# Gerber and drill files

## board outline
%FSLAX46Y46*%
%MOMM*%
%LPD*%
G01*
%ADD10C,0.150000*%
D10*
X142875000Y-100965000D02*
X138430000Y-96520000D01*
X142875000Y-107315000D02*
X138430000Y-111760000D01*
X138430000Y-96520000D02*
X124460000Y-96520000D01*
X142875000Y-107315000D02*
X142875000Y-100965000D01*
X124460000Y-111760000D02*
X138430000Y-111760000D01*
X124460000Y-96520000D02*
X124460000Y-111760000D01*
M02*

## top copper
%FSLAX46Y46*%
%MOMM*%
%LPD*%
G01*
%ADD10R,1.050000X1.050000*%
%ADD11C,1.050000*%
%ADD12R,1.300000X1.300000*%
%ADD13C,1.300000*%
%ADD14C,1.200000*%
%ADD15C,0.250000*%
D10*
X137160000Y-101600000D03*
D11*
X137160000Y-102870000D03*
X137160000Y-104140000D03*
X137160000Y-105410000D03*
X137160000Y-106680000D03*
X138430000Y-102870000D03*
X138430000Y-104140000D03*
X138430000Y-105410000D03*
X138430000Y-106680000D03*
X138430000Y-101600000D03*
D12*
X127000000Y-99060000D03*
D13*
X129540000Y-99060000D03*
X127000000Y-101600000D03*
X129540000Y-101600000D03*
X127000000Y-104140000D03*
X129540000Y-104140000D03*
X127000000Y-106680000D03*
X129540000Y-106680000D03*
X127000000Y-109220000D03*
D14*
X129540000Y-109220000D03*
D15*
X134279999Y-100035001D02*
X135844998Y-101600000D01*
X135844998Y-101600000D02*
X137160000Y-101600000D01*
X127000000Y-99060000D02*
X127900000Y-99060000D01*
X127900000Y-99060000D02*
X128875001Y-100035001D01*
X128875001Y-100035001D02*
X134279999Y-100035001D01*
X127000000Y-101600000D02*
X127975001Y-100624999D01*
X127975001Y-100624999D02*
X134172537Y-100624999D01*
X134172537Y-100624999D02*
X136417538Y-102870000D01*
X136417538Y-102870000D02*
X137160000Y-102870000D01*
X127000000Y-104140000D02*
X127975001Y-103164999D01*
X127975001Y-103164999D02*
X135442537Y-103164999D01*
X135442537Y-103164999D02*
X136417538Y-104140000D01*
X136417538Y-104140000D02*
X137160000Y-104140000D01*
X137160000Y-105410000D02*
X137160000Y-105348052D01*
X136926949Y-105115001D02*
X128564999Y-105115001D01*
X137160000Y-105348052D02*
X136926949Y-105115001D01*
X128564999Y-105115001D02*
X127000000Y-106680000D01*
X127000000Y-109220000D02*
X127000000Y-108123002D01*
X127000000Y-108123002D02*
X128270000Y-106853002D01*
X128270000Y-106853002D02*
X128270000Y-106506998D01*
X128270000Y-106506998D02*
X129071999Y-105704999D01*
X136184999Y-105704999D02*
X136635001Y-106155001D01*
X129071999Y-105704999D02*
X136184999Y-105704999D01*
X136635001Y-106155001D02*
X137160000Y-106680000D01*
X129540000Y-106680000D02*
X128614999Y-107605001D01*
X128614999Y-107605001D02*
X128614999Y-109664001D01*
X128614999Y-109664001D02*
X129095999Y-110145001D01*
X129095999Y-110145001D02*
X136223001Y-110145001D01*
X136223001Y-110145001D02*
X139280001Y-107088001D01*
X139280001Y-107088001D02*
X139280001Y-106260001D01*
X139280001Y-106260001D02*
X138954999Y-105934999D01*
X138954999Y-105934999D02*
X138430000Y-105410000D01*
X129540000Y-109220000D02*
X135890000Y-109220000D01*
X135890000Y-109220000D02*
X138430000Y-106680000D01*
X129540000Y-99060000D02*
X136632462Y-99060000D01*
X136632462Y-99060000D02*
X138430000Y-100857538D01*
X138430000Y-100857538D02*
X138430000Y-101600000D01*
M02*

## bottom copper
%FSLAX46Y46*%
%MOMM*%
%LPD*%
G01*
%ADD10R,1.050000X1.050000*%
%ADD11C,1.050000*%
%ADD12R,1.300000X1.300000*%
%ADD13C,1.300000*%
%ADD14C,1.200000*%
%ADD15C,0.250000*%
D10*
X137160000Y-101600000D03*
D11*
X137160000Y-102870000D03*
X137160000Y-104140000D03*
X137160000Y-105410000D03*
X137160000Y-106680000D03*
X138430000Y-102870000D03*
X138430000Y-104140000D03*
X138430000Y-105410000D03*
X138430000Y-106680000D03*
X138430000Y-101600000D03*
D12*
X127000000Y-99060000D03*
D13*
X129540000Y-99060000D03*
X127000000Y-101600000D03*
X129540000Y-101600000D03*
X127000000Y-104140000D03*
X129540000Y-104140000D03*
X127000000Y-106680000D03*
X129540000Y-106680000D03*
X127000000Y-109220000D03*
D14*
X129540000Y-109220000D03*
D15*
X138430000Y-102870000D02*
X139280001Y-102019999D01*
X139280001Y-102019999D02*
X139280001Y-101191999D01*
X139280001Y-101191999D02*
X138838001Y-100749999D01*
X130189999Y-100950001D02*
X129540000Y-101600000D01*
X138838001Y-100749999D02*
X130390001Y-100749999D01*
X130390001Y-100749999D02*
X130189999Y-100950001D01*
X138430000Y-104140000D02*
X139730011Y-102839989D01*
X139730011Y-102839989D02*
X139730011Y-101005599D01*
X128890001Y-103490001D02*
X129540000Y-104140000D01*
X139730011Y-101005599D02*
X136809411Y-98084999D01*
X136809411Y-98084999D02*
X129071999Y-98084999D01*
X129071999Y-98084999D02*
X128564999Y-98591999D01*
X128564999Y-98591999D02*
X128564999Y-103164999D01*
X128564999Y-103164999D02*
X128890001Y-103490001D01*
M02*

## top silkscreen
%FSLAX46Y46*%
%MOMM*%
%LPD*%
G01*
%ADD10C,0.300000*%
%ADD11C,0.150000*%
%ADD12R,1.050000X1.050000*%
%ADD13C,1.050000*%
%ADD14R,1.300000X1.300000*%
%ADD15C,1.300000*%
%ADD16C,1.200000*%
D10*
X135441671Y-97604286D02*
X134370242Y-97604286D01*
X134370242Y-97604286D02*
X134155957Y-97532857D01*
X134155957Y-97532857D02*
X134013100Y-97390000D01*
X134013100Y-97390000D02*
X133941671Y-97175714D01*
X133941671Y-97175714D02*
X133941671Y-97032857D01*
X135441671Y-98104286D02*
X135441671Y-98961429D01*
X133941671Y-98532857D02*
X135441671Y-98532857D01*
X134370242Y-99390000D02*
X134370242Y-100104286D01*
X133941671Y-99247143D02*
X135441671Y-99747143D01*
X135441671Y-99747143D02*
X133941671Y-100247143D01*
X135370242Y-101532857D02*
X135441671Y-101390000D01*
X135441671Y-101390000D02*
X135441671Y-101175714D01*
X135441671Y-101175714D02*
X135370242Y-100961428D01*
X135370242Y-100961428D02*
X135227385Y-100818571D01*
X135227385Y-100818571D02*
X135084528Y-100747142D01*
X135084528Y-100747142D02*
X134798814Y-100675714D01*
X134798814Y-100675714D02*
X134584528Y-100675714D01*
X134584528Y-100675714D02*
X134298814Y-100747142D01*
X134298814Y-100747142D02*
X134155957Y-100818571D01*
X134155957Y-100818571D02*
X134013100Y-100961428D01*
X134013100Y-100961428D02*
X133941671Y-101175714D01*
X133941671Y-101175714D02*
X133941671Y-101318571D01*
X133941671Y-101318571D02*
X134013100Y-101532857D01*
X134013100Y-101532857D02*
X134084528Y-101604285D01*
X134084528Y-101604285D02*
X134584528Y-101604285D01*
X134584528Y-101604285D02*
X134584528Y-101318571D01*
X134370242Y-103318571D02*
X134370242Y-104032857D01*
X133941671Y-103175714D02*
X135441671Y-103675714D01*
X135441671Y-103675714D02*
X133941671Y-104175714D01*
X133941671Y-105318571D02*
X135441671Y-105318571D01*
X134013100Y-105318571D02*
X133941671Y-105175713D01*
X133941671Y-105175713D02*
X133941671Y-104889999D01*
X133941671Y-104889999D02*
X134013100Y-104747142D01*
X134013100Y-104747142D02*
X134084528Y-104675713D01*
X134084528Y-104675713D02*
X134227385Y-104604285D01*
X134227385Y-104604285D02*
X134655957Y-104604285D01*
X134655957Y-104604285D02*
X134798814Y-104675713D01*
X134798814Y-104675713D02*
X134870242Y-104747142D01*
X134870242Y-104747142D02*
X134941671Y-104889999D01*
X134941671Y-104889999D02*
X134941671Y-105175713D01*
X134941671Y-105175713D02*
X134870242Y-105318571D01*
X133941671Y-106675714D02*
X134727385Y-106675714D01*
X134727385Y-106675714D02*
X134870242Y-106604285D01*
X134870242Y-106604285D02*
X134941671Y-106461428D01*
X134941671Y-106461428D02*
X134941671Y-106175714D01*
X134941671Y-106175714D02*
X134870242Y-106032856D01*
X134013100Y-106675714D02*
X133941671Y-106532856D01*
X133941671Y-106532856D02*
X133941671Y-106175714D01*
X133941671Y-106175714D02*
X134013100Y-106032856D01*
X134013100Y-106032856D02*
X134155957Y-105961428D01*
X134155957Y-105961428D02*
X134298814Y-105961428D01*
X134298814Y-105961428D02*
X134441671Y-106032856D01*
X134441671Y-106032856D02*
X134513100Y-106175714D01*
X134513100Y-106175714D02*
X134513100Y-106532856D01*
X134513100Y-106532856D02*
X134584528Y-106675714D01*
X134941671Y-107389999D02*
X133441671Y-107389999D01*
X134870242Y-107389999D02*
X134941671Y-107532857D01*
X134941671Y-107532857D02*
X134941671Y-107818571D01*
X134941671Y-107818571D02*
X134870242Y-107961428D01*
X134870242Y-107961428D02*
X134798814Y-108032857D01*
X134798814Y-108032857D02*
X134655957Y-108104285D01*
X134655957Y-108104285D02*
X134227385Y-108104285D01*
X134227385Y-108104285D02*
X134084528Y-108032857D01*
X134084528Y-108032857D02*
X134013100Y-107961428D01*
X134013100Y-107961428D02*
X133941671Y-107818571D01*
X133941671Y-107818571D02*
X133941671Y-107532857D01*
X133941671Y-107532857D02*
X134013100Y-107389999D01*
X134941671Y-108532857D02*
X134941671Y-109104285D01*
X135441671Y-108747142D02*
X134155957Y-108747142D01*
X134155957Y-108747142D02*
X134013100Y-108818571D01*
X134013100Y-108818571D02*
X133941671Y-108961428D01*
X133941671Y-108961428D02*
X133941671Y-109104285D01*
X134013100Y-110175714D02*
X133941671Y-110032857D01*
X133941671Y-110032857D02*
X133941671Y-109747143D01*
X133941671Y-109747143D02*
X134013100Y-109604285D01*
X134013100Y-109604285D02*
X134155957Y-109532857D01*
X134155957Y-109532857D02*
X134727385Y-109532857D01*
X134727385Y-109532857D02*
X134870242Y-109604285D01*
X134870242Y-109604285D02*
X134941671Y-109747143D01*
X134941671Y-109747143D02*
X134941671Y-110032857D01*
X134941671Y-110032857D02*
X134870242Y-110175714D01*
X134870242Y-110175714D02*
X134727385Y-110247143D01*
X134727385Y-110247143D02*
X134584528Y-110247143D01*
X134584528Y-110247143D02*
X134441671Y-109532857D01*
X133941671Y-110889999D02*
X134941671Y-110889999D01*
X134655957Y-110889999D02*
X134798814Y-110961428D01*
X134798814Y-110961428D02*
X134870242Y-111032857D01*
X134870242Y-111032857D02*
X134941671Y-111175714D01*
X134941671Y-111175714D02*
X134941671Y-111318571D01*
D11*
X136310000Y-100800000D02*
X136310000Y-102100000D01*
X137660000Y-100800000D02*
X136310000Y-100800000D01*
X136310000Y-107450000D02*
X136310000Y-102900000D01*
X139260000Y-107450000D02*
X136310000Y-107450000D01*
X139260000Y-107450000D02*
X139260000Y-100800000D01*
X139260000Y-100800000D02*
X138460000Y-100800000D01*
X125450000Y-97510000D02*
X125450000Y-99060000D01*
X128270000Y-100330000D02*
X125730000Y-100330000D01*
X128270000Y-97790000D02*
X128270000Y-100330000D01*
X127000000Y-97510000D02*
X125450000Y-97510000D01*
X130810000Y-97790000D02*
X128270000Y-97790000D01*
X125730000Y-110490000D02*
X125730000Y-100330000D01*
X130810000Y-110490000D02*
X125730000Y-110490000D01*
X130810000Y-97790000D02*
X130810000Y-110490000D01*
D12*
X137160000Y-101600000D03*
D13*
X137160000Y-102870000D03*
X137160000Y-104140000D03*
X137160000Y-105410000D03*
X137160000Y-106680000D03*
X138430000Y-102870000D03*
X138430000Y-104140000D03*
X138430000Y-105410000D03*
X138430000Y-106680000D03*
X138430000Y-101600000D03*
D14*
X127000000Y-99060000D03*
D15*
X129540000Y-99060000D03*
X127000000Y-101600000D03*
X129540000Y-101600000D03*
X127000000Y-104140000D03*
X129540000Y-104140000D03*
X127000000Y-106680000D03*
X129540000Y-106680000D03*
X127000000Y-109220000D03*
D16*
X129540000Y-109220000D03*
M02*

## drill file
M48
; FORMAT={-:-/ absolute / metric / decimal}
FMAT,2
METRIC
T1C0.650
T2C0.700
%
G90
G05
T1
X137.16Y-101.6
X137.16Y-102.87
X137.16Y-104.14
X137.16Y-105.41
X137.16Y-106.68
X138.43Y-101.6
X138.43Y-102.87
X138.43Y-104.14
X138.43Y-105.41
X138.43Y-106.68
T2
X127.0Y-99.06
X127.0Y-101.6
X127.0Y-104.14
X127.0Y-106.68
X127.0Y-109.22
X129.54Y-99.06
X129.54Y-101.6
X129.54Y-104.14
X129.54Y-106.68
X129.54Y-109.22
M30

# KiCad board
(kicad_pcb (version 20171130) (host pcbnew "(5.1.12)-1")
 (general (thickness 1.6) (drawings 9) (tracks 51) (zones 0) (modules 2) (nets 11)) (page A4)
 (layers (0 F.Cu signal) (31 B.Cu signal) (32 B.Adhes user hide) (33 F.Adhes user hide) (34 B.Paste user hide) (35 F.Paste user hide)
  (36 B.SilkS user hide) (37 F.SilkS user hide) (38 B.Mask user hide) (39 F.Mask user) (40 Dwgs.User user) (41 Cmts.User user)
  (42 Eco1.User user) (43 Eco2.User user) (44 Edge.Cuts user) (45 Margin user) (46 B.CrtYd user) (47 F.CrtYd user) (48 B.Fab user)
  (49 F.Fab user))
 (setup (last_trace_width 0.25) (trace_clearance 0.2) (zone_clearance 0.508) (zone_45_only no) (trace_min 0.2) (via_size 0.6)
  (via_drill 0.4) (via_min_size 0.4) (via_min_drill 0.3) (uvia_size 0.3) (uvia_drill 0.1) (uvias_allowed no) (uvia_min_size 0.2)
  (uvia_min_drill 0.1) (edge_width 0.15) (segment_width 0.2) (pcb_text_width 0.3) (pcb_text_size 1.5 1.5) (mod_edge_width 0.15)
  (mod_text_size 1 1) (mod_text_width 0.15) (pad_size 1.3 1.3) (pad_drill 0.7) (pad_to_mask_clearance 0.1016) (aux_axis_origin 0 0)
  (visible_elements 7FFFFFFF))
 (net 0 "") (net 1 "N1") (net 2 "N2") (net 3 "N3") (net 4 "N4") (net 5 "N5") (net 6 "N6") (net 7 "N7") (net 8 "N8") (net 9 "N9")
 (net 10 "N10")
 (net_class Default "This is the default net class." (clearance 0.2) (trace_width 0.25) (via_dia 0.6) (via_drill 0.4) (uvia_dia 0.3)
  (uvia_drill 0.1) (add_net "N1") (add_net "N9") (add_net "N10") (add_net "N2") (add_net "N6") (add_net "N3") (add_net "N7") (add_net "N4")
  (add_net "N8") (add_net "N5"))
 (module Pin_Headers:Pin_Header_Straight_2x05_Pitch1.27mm (layer F.Cu) (at 137.16 101.6)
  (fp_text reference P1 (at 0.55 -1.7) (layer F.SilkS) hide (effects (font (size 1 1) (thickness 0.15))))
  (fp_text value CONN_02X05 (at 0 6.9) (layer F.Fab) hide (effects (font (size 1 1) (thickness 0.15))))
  (fp_line (start -0.85 -0.8) (end -0.85 0.5) (layer F.SilkS) (width 0.15))
  (fp_line (start 0.5 -0.8) (end -0.85 -0.8) (layer F.SilkS) (width 0.15))
  (fp_line (start -0.85 5.85) (end -0.85 1.3) (layer F.SilkS) (width 0.15))
  (fp_line (start 2.1 5.85) (end -0.85 5.85) (layer F.SilkS) (width 0.15))
  (fp_line (start 2.1 5.85) (end 2.1 -0.8) (layer F.SilkS) (width 0.15))
  (fp_line (start 2.1 -0.8) (end 1.3 -0.8) (layer F.SilkS) (width 0.15))
  (pad 1 thru_hole rect (at 0 0) (size 1.05 1.05) (drill 0.65) (layers *.Cu *.Mask F.SilkS) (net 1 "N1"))
  (pad 3 thru_hole circle (at 0 1.27) (size 1.05 1.05) (drill 0.65) (layers *.Cu *.Mask F.SilkS) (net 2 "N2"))
  (pad 5 thru_hole circle (at 0 2.54) (size 1.05 1.05) (drill 0.65) (layers *.Cu *.Mask F.SilkS) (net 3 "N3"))
  (pad 7 thru_hole circle (at 0 3.81) (size 1.05 1.05) (drill 0.65) (layers *.Cu *.Mask F.SilkS) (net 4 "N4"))
  (pad 9 thru_hole circle (at 0 5.08) (size 1.05 1.05) (drill 0.65) (layers *.Cu *.Mask F.SilkS) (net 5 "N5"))
  (pad 4 thru_hole circle (at 1.27 1.27) (size 1.05 1.05) (drill 0.65) (layers *.Cu *.Mask F.SilkS) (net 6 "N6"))
  (pad 6 thru_hole circle (at 1.27 2.54) (size 1.05 1.05) (drill 0.65) (layers *.Cu *.Mask F.SilkS) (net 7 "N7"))
  (pad 8 thru_hole circle (at 1.27 3.81) (size 1.05 1.05) (drill 0.65) (layers *.Cu *.Mask F.SilkS) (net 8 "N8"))
  (pad 10 thru_hole circle (at 1.27 5.08) (size 1.05 1.05) (drill 0.65) (layers *.Cu *.Mask F.SilkS) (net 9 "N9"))
  (pad 2 thru_hole circle (at 1.27 0) (size 1.05 1.05) (drill 0.65) (layers *.Cu *.Mask F.SilkS) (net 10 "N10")))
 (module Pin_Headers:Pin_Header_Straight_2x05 (layer F.Cu) (at 127 99.06)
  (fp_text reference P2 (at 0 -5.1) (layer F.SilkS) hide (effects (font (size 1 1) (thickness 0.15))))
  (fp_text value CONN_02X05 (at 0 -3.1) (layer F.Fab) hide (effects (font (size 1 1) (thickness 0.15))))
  (fp_line (start -1.55 -1.55) (end -1.55 0) (layer F.SilkS) (width 0.15))
  (fp_line (start 1.27 1.27) (end -1.27 1.27) (layer F.SilkS) (width 0.15))
  (fp_line (start 1.27 -1.27) (end 1.27 1.27) (layer F.SilkS) (width 0.15))
  (fp_line (start 0 -1.55) (end -1.55 -1.55) (layer F.SilkS) (width 0.15))
  (fp_line (start 3.81 -1.27) (end 1.27 -1.27) (layer F.SilkS) (width 0.15))
  (fp_line (start -1.27 11.43) (end -1.27 1.27) (layer F.SilkS) (width 0.15))
  (fp_line (start 3.81 11.43) (end -1.27 11.43) (layer F.SilkS) (width 0.15))
  (fp_line (start 3.81 -1.27) (end 3.81 11.43) (layer F.SilkS) (width 0.15))
  (pad 1 thru_hole rect (at 0 0) (size 1.3 1.3) (drill 0.7) (layers *.Cu *.Mask F.SilkS) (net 1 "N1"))
  (pad 2 thru_hole circle (at 2.54 0) (size 1.3 1.3) (drill 0.7) (layers *.Cu *.Mask F.SilkS) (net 10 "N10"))
  (pad 3 thru_hole circle (at 0 2.54) (size 1.3 1.3) (drill 0.7) (layers *.Cu *.Mask F.SilkS) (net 2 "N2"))
  (pad 4 thru_hole circle (at 2.54 2.54) (size 1.3 1.3) (drill 0.7) (layers *.Cu *.Mask F.SilkS) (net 6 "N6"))
  (pad 5 thru_hole circle (at 0 5.08) (size 1.3 1.3) (drill 0.7) (layers *.Cu *.Mask F.SilkS) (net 3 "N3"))
  (pad 6 thru_hole circle (at 2.54 5.08) (size 1.3 1.3) (drill 0.7) (layers *.Cu *.Mask F.SilkS) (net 7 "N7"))
  (pad 7 thru_hole circle (at 0 7.62) (size 1.3 1.3) (drill 0.7) (layers *.Cu *.Mask F.SilkS) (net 4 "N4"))
  (pad 8 thru_hole circle (at 2.54 7.62) (size 1.3 1.3) (drill 0.7) (layers *.Cu *.Mask F.SilkS) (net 8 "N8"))
  (pad 9 thru_hole circle (at 0 10.16) (size 1.3 1.3) (drill 0.7) (layers *.Cu *.Mask F.SilkS) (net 5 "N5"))
  (pad 10 thru_hole circle (at 2.54 10.16) (size 1.2 1.2) (drill 0.7) (layers *.Cu *.Mask F.SilkS) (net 9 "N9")))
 (gr_line (start 142.875 100.965) (end 138.43 96.52) (layer Edge.Cuts) (width 0.15))
 (gr_line (start 142.875 107.315) (end 138.43 111.76) (layer Edge.Cuts) (width 0.15))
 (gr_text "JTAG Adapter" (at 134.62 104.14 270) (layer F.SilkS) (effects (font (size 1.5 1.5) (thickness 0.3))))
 (gr_line (start 138.43 96.52) (end 124.46 96.52) (layer Edge.Cuts) (width 0.15))
 (gr_line (start 142.875 107.315) (end 142.875 100.965) (layer Edge.Cuts) (width 0.15))
 (gr_line (start 124.46 111.76) (end 138.43 111.76) (layer Edge.Cuts) (width 0.15))
 (gr_line (start 124.46 96.52) (end 124.46 111.76) (layer Edge.Cuts) (width 0.15))
 (segment (start 134.279999 100.035001) (end 135.844998 101.6) (width 0.25) (layer F.Cu) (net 1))
 (segment (start 135.844998 101.6) (end 137.16 101.6) (width 0.25) (layer F.Cu) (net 1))
 (segment (start 127 99.06) (end 127.9 99.06) (width 0.25) (layer F.Cu) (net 1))
 (segment (start 127.9 99.06) (end 128.875001 100.035001) (width 0.25) (layer F.Cu) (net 1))
 (segment (start 128.875001 100.035001) (end 134.279999 100.035001) (width 0.25) (layer F.Cu) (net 1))
 (segment (start 127 101.6) (end 127.975001 100.624999) (width 0.25) (layer F.Cu) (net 2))
 (segment (start 127.975001 100.624999) (end 134.172537 100.624999) (width 0.25) (layer F.Cu) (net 2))
 (segment (start 134.172537 100.624999) (end 136.417538 102.87) (width 0.25) (layer F.Cu) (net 2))
 (segment (start 136.417538 102.87) (end 137.16 102.87) (width 0.25) (layer F.Cu) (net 2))
 (segment (start 127 104.14) (end 127.975001 103.164999) (width 0.25) (layer F.Cu) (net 3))
 (segment (start 127.975001 103.164999) (end 135.442537 103.164999) (width 0.25) (layer F.Cu) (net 3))
 (segment (start 135.442537 103.164999) (end 136.417538 104.14) (width 0.25) (layer F.Cu) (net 3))
 (segment (start 136.417538 104.14) (end 137.16 104.14) (width 0.25) (layer F.Cu) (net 3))
 (segment (start 137.16 105.41) (end 137.16 105.348052) (width 0.25) (layer F.Cu) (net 4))
 (segment (start 136.926949 105.115001) (end 128.564999 105.115001) (width 0.25) (layer F.Cu) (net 4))
 (segment (start 137.16 105.348052) (end 136.926949 105.115001) (width 0.25) (layer F.Cu) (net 4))
 (segment (start 128.564999 105.115001) (end 127 106.68) (width 0.25) (layer F.Cu) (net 4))
 (segment (start 127 109.22) (end 127 108.123002) (width 0.25) (layer F.Cu) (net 5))
 (segment (start 127 108.123002) (end 128.27 106.853002) (width 0.25) (layer F.Cu) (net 5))
 (segment (start 128.27 106.853002) (end 128.27 106.506998) (width 0.25) (layer F.Cu) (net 5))
 (segment (start 128.27 106.506998) (end 129.071999 105.704999) (width 0.25) (layer F.Cu) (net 5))
 (segment (start 136.184999 105.704999) (end 136.635001 106.155001) (width 0.25) (layer F.Cu) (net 5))
 (segment (start 129.071999 105.704999) (end 136.184999 105.704999) (width 0.25) (layer F.Cu) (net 5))
 (segment (start 136.635001 106.155001) (end 137.16 106.68) (width 0.25) (layer F.Cu) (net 5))
 (segment (start 138.43 102.87) (end 139.280001 102.019999) (width 0.25) (layer B.Cu) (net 6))
 (segment (start 139.280001 102.019999) (end 139.280001 101.191999) (width 0.25) (layer B.Cu) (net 6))
 (segment (start 139.280001 101.191999) (end 138.838001 100.749999) (width 0.25) (layer B.Cu) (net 6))
 (segment (start 130.189999 100.950001) (end 129.54 101.6) (width 0.25) (layer B.Cu) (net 6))
 (segment (start 138.838001 100.749999) (end 130.390001 100.749999) (width 0.25) (layer B.Cu) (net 6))
 (segment (start 130.390001 100.749999) (end 130.189999 100.950001) (width 0.25) (layer B.Cu) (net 6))
 (segment (start 138.43 104.14) (end 139.730011 102.839989) (width 0.25) (layer B.Cu) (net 7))
 (segment (start 139.730011 102.839989) (end 139.730011 101.005599) (width 0.25) (layer B.Cu) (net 7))
 (segment (start 128.890001 103.490001) (end 129.54 104.14) (width 0.25) (layer B.Cu) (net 7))
 (segment (start 139.730011 101.005599) (end 136.809411 98.084999) (width 0.25) (layer B.Cu) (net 7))
 (segment (start 136.809411 98.084999) (end 129.071999 98.084999) (width 0.25) (layer B.Cu) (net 7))
 (segment (start 129.071999 98.084999) (end 128.564999 98.591999) (width 0.25) (layer B.Cu) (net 7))
 (segment (start 128.564999 98.591999) (end 128.564999 103.164999) (width 0.25) (layer B.Cu) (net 7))
 (segment (start 128.564999 103.164999) (end 128.890001 103.490001) (width 0.25) (layer B.Cu) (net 7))
 (segment (start 129.54 106.68) (end 128.614999 107.605001) (width 0.25) (layer F.Cu) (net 8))
 (segment (start 128.614999 107.605001) (end 128.614999 109.664001) (width 0.25) (layer F.Cu) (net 8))
 (segment (start 128.614999 109.664001) (end 129.095999 110.145001) (width 0.25) (layer F.Cu) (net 8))
 (segment (start 129.095999 110.145001) (end 136.223001 110.145001) (width 0.25) (layer F.Cu) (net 8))
 (segment (start 136.223001 110.145001) (end 139.280001 107.088001) (width 0.25) (layer F.Cu) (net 8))
 (segment (start 139.280001 107.088001) (end 139.280001 106.260001) (width 0.25) (layer F.Cu) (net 8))
 (segment (start 139.280001 106.260001) (end 138.954999 105.934999) (width 0.25) (layer F.Cu) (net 8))
 (segment (start 138.954999 105.934999) (end 138.43 105.41) (width 0.25) (layer F.Cu) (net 8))
 (segment (start 129.54 109.22) (end 135.89 109.22) (width 0.25) (layer F.Cu) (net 9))
 (segment (start 135.89 109.22) (end 138.43 106.68) (width 0.25) (layer F.Cu) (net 9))
 (segment (start 129.54 99.06) (end 136.632462 99.06) (width 0.25) (layer F.Cu) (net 10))
 (segment (start 136.632462 99.06) (end 138.43 100.857538) (width 0.25) (layer F.Cu) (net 10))
 (segment (start 138.43 100.857538) (end 138.43 101.6) (width 0.25) (layer F.Cu) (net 10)))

